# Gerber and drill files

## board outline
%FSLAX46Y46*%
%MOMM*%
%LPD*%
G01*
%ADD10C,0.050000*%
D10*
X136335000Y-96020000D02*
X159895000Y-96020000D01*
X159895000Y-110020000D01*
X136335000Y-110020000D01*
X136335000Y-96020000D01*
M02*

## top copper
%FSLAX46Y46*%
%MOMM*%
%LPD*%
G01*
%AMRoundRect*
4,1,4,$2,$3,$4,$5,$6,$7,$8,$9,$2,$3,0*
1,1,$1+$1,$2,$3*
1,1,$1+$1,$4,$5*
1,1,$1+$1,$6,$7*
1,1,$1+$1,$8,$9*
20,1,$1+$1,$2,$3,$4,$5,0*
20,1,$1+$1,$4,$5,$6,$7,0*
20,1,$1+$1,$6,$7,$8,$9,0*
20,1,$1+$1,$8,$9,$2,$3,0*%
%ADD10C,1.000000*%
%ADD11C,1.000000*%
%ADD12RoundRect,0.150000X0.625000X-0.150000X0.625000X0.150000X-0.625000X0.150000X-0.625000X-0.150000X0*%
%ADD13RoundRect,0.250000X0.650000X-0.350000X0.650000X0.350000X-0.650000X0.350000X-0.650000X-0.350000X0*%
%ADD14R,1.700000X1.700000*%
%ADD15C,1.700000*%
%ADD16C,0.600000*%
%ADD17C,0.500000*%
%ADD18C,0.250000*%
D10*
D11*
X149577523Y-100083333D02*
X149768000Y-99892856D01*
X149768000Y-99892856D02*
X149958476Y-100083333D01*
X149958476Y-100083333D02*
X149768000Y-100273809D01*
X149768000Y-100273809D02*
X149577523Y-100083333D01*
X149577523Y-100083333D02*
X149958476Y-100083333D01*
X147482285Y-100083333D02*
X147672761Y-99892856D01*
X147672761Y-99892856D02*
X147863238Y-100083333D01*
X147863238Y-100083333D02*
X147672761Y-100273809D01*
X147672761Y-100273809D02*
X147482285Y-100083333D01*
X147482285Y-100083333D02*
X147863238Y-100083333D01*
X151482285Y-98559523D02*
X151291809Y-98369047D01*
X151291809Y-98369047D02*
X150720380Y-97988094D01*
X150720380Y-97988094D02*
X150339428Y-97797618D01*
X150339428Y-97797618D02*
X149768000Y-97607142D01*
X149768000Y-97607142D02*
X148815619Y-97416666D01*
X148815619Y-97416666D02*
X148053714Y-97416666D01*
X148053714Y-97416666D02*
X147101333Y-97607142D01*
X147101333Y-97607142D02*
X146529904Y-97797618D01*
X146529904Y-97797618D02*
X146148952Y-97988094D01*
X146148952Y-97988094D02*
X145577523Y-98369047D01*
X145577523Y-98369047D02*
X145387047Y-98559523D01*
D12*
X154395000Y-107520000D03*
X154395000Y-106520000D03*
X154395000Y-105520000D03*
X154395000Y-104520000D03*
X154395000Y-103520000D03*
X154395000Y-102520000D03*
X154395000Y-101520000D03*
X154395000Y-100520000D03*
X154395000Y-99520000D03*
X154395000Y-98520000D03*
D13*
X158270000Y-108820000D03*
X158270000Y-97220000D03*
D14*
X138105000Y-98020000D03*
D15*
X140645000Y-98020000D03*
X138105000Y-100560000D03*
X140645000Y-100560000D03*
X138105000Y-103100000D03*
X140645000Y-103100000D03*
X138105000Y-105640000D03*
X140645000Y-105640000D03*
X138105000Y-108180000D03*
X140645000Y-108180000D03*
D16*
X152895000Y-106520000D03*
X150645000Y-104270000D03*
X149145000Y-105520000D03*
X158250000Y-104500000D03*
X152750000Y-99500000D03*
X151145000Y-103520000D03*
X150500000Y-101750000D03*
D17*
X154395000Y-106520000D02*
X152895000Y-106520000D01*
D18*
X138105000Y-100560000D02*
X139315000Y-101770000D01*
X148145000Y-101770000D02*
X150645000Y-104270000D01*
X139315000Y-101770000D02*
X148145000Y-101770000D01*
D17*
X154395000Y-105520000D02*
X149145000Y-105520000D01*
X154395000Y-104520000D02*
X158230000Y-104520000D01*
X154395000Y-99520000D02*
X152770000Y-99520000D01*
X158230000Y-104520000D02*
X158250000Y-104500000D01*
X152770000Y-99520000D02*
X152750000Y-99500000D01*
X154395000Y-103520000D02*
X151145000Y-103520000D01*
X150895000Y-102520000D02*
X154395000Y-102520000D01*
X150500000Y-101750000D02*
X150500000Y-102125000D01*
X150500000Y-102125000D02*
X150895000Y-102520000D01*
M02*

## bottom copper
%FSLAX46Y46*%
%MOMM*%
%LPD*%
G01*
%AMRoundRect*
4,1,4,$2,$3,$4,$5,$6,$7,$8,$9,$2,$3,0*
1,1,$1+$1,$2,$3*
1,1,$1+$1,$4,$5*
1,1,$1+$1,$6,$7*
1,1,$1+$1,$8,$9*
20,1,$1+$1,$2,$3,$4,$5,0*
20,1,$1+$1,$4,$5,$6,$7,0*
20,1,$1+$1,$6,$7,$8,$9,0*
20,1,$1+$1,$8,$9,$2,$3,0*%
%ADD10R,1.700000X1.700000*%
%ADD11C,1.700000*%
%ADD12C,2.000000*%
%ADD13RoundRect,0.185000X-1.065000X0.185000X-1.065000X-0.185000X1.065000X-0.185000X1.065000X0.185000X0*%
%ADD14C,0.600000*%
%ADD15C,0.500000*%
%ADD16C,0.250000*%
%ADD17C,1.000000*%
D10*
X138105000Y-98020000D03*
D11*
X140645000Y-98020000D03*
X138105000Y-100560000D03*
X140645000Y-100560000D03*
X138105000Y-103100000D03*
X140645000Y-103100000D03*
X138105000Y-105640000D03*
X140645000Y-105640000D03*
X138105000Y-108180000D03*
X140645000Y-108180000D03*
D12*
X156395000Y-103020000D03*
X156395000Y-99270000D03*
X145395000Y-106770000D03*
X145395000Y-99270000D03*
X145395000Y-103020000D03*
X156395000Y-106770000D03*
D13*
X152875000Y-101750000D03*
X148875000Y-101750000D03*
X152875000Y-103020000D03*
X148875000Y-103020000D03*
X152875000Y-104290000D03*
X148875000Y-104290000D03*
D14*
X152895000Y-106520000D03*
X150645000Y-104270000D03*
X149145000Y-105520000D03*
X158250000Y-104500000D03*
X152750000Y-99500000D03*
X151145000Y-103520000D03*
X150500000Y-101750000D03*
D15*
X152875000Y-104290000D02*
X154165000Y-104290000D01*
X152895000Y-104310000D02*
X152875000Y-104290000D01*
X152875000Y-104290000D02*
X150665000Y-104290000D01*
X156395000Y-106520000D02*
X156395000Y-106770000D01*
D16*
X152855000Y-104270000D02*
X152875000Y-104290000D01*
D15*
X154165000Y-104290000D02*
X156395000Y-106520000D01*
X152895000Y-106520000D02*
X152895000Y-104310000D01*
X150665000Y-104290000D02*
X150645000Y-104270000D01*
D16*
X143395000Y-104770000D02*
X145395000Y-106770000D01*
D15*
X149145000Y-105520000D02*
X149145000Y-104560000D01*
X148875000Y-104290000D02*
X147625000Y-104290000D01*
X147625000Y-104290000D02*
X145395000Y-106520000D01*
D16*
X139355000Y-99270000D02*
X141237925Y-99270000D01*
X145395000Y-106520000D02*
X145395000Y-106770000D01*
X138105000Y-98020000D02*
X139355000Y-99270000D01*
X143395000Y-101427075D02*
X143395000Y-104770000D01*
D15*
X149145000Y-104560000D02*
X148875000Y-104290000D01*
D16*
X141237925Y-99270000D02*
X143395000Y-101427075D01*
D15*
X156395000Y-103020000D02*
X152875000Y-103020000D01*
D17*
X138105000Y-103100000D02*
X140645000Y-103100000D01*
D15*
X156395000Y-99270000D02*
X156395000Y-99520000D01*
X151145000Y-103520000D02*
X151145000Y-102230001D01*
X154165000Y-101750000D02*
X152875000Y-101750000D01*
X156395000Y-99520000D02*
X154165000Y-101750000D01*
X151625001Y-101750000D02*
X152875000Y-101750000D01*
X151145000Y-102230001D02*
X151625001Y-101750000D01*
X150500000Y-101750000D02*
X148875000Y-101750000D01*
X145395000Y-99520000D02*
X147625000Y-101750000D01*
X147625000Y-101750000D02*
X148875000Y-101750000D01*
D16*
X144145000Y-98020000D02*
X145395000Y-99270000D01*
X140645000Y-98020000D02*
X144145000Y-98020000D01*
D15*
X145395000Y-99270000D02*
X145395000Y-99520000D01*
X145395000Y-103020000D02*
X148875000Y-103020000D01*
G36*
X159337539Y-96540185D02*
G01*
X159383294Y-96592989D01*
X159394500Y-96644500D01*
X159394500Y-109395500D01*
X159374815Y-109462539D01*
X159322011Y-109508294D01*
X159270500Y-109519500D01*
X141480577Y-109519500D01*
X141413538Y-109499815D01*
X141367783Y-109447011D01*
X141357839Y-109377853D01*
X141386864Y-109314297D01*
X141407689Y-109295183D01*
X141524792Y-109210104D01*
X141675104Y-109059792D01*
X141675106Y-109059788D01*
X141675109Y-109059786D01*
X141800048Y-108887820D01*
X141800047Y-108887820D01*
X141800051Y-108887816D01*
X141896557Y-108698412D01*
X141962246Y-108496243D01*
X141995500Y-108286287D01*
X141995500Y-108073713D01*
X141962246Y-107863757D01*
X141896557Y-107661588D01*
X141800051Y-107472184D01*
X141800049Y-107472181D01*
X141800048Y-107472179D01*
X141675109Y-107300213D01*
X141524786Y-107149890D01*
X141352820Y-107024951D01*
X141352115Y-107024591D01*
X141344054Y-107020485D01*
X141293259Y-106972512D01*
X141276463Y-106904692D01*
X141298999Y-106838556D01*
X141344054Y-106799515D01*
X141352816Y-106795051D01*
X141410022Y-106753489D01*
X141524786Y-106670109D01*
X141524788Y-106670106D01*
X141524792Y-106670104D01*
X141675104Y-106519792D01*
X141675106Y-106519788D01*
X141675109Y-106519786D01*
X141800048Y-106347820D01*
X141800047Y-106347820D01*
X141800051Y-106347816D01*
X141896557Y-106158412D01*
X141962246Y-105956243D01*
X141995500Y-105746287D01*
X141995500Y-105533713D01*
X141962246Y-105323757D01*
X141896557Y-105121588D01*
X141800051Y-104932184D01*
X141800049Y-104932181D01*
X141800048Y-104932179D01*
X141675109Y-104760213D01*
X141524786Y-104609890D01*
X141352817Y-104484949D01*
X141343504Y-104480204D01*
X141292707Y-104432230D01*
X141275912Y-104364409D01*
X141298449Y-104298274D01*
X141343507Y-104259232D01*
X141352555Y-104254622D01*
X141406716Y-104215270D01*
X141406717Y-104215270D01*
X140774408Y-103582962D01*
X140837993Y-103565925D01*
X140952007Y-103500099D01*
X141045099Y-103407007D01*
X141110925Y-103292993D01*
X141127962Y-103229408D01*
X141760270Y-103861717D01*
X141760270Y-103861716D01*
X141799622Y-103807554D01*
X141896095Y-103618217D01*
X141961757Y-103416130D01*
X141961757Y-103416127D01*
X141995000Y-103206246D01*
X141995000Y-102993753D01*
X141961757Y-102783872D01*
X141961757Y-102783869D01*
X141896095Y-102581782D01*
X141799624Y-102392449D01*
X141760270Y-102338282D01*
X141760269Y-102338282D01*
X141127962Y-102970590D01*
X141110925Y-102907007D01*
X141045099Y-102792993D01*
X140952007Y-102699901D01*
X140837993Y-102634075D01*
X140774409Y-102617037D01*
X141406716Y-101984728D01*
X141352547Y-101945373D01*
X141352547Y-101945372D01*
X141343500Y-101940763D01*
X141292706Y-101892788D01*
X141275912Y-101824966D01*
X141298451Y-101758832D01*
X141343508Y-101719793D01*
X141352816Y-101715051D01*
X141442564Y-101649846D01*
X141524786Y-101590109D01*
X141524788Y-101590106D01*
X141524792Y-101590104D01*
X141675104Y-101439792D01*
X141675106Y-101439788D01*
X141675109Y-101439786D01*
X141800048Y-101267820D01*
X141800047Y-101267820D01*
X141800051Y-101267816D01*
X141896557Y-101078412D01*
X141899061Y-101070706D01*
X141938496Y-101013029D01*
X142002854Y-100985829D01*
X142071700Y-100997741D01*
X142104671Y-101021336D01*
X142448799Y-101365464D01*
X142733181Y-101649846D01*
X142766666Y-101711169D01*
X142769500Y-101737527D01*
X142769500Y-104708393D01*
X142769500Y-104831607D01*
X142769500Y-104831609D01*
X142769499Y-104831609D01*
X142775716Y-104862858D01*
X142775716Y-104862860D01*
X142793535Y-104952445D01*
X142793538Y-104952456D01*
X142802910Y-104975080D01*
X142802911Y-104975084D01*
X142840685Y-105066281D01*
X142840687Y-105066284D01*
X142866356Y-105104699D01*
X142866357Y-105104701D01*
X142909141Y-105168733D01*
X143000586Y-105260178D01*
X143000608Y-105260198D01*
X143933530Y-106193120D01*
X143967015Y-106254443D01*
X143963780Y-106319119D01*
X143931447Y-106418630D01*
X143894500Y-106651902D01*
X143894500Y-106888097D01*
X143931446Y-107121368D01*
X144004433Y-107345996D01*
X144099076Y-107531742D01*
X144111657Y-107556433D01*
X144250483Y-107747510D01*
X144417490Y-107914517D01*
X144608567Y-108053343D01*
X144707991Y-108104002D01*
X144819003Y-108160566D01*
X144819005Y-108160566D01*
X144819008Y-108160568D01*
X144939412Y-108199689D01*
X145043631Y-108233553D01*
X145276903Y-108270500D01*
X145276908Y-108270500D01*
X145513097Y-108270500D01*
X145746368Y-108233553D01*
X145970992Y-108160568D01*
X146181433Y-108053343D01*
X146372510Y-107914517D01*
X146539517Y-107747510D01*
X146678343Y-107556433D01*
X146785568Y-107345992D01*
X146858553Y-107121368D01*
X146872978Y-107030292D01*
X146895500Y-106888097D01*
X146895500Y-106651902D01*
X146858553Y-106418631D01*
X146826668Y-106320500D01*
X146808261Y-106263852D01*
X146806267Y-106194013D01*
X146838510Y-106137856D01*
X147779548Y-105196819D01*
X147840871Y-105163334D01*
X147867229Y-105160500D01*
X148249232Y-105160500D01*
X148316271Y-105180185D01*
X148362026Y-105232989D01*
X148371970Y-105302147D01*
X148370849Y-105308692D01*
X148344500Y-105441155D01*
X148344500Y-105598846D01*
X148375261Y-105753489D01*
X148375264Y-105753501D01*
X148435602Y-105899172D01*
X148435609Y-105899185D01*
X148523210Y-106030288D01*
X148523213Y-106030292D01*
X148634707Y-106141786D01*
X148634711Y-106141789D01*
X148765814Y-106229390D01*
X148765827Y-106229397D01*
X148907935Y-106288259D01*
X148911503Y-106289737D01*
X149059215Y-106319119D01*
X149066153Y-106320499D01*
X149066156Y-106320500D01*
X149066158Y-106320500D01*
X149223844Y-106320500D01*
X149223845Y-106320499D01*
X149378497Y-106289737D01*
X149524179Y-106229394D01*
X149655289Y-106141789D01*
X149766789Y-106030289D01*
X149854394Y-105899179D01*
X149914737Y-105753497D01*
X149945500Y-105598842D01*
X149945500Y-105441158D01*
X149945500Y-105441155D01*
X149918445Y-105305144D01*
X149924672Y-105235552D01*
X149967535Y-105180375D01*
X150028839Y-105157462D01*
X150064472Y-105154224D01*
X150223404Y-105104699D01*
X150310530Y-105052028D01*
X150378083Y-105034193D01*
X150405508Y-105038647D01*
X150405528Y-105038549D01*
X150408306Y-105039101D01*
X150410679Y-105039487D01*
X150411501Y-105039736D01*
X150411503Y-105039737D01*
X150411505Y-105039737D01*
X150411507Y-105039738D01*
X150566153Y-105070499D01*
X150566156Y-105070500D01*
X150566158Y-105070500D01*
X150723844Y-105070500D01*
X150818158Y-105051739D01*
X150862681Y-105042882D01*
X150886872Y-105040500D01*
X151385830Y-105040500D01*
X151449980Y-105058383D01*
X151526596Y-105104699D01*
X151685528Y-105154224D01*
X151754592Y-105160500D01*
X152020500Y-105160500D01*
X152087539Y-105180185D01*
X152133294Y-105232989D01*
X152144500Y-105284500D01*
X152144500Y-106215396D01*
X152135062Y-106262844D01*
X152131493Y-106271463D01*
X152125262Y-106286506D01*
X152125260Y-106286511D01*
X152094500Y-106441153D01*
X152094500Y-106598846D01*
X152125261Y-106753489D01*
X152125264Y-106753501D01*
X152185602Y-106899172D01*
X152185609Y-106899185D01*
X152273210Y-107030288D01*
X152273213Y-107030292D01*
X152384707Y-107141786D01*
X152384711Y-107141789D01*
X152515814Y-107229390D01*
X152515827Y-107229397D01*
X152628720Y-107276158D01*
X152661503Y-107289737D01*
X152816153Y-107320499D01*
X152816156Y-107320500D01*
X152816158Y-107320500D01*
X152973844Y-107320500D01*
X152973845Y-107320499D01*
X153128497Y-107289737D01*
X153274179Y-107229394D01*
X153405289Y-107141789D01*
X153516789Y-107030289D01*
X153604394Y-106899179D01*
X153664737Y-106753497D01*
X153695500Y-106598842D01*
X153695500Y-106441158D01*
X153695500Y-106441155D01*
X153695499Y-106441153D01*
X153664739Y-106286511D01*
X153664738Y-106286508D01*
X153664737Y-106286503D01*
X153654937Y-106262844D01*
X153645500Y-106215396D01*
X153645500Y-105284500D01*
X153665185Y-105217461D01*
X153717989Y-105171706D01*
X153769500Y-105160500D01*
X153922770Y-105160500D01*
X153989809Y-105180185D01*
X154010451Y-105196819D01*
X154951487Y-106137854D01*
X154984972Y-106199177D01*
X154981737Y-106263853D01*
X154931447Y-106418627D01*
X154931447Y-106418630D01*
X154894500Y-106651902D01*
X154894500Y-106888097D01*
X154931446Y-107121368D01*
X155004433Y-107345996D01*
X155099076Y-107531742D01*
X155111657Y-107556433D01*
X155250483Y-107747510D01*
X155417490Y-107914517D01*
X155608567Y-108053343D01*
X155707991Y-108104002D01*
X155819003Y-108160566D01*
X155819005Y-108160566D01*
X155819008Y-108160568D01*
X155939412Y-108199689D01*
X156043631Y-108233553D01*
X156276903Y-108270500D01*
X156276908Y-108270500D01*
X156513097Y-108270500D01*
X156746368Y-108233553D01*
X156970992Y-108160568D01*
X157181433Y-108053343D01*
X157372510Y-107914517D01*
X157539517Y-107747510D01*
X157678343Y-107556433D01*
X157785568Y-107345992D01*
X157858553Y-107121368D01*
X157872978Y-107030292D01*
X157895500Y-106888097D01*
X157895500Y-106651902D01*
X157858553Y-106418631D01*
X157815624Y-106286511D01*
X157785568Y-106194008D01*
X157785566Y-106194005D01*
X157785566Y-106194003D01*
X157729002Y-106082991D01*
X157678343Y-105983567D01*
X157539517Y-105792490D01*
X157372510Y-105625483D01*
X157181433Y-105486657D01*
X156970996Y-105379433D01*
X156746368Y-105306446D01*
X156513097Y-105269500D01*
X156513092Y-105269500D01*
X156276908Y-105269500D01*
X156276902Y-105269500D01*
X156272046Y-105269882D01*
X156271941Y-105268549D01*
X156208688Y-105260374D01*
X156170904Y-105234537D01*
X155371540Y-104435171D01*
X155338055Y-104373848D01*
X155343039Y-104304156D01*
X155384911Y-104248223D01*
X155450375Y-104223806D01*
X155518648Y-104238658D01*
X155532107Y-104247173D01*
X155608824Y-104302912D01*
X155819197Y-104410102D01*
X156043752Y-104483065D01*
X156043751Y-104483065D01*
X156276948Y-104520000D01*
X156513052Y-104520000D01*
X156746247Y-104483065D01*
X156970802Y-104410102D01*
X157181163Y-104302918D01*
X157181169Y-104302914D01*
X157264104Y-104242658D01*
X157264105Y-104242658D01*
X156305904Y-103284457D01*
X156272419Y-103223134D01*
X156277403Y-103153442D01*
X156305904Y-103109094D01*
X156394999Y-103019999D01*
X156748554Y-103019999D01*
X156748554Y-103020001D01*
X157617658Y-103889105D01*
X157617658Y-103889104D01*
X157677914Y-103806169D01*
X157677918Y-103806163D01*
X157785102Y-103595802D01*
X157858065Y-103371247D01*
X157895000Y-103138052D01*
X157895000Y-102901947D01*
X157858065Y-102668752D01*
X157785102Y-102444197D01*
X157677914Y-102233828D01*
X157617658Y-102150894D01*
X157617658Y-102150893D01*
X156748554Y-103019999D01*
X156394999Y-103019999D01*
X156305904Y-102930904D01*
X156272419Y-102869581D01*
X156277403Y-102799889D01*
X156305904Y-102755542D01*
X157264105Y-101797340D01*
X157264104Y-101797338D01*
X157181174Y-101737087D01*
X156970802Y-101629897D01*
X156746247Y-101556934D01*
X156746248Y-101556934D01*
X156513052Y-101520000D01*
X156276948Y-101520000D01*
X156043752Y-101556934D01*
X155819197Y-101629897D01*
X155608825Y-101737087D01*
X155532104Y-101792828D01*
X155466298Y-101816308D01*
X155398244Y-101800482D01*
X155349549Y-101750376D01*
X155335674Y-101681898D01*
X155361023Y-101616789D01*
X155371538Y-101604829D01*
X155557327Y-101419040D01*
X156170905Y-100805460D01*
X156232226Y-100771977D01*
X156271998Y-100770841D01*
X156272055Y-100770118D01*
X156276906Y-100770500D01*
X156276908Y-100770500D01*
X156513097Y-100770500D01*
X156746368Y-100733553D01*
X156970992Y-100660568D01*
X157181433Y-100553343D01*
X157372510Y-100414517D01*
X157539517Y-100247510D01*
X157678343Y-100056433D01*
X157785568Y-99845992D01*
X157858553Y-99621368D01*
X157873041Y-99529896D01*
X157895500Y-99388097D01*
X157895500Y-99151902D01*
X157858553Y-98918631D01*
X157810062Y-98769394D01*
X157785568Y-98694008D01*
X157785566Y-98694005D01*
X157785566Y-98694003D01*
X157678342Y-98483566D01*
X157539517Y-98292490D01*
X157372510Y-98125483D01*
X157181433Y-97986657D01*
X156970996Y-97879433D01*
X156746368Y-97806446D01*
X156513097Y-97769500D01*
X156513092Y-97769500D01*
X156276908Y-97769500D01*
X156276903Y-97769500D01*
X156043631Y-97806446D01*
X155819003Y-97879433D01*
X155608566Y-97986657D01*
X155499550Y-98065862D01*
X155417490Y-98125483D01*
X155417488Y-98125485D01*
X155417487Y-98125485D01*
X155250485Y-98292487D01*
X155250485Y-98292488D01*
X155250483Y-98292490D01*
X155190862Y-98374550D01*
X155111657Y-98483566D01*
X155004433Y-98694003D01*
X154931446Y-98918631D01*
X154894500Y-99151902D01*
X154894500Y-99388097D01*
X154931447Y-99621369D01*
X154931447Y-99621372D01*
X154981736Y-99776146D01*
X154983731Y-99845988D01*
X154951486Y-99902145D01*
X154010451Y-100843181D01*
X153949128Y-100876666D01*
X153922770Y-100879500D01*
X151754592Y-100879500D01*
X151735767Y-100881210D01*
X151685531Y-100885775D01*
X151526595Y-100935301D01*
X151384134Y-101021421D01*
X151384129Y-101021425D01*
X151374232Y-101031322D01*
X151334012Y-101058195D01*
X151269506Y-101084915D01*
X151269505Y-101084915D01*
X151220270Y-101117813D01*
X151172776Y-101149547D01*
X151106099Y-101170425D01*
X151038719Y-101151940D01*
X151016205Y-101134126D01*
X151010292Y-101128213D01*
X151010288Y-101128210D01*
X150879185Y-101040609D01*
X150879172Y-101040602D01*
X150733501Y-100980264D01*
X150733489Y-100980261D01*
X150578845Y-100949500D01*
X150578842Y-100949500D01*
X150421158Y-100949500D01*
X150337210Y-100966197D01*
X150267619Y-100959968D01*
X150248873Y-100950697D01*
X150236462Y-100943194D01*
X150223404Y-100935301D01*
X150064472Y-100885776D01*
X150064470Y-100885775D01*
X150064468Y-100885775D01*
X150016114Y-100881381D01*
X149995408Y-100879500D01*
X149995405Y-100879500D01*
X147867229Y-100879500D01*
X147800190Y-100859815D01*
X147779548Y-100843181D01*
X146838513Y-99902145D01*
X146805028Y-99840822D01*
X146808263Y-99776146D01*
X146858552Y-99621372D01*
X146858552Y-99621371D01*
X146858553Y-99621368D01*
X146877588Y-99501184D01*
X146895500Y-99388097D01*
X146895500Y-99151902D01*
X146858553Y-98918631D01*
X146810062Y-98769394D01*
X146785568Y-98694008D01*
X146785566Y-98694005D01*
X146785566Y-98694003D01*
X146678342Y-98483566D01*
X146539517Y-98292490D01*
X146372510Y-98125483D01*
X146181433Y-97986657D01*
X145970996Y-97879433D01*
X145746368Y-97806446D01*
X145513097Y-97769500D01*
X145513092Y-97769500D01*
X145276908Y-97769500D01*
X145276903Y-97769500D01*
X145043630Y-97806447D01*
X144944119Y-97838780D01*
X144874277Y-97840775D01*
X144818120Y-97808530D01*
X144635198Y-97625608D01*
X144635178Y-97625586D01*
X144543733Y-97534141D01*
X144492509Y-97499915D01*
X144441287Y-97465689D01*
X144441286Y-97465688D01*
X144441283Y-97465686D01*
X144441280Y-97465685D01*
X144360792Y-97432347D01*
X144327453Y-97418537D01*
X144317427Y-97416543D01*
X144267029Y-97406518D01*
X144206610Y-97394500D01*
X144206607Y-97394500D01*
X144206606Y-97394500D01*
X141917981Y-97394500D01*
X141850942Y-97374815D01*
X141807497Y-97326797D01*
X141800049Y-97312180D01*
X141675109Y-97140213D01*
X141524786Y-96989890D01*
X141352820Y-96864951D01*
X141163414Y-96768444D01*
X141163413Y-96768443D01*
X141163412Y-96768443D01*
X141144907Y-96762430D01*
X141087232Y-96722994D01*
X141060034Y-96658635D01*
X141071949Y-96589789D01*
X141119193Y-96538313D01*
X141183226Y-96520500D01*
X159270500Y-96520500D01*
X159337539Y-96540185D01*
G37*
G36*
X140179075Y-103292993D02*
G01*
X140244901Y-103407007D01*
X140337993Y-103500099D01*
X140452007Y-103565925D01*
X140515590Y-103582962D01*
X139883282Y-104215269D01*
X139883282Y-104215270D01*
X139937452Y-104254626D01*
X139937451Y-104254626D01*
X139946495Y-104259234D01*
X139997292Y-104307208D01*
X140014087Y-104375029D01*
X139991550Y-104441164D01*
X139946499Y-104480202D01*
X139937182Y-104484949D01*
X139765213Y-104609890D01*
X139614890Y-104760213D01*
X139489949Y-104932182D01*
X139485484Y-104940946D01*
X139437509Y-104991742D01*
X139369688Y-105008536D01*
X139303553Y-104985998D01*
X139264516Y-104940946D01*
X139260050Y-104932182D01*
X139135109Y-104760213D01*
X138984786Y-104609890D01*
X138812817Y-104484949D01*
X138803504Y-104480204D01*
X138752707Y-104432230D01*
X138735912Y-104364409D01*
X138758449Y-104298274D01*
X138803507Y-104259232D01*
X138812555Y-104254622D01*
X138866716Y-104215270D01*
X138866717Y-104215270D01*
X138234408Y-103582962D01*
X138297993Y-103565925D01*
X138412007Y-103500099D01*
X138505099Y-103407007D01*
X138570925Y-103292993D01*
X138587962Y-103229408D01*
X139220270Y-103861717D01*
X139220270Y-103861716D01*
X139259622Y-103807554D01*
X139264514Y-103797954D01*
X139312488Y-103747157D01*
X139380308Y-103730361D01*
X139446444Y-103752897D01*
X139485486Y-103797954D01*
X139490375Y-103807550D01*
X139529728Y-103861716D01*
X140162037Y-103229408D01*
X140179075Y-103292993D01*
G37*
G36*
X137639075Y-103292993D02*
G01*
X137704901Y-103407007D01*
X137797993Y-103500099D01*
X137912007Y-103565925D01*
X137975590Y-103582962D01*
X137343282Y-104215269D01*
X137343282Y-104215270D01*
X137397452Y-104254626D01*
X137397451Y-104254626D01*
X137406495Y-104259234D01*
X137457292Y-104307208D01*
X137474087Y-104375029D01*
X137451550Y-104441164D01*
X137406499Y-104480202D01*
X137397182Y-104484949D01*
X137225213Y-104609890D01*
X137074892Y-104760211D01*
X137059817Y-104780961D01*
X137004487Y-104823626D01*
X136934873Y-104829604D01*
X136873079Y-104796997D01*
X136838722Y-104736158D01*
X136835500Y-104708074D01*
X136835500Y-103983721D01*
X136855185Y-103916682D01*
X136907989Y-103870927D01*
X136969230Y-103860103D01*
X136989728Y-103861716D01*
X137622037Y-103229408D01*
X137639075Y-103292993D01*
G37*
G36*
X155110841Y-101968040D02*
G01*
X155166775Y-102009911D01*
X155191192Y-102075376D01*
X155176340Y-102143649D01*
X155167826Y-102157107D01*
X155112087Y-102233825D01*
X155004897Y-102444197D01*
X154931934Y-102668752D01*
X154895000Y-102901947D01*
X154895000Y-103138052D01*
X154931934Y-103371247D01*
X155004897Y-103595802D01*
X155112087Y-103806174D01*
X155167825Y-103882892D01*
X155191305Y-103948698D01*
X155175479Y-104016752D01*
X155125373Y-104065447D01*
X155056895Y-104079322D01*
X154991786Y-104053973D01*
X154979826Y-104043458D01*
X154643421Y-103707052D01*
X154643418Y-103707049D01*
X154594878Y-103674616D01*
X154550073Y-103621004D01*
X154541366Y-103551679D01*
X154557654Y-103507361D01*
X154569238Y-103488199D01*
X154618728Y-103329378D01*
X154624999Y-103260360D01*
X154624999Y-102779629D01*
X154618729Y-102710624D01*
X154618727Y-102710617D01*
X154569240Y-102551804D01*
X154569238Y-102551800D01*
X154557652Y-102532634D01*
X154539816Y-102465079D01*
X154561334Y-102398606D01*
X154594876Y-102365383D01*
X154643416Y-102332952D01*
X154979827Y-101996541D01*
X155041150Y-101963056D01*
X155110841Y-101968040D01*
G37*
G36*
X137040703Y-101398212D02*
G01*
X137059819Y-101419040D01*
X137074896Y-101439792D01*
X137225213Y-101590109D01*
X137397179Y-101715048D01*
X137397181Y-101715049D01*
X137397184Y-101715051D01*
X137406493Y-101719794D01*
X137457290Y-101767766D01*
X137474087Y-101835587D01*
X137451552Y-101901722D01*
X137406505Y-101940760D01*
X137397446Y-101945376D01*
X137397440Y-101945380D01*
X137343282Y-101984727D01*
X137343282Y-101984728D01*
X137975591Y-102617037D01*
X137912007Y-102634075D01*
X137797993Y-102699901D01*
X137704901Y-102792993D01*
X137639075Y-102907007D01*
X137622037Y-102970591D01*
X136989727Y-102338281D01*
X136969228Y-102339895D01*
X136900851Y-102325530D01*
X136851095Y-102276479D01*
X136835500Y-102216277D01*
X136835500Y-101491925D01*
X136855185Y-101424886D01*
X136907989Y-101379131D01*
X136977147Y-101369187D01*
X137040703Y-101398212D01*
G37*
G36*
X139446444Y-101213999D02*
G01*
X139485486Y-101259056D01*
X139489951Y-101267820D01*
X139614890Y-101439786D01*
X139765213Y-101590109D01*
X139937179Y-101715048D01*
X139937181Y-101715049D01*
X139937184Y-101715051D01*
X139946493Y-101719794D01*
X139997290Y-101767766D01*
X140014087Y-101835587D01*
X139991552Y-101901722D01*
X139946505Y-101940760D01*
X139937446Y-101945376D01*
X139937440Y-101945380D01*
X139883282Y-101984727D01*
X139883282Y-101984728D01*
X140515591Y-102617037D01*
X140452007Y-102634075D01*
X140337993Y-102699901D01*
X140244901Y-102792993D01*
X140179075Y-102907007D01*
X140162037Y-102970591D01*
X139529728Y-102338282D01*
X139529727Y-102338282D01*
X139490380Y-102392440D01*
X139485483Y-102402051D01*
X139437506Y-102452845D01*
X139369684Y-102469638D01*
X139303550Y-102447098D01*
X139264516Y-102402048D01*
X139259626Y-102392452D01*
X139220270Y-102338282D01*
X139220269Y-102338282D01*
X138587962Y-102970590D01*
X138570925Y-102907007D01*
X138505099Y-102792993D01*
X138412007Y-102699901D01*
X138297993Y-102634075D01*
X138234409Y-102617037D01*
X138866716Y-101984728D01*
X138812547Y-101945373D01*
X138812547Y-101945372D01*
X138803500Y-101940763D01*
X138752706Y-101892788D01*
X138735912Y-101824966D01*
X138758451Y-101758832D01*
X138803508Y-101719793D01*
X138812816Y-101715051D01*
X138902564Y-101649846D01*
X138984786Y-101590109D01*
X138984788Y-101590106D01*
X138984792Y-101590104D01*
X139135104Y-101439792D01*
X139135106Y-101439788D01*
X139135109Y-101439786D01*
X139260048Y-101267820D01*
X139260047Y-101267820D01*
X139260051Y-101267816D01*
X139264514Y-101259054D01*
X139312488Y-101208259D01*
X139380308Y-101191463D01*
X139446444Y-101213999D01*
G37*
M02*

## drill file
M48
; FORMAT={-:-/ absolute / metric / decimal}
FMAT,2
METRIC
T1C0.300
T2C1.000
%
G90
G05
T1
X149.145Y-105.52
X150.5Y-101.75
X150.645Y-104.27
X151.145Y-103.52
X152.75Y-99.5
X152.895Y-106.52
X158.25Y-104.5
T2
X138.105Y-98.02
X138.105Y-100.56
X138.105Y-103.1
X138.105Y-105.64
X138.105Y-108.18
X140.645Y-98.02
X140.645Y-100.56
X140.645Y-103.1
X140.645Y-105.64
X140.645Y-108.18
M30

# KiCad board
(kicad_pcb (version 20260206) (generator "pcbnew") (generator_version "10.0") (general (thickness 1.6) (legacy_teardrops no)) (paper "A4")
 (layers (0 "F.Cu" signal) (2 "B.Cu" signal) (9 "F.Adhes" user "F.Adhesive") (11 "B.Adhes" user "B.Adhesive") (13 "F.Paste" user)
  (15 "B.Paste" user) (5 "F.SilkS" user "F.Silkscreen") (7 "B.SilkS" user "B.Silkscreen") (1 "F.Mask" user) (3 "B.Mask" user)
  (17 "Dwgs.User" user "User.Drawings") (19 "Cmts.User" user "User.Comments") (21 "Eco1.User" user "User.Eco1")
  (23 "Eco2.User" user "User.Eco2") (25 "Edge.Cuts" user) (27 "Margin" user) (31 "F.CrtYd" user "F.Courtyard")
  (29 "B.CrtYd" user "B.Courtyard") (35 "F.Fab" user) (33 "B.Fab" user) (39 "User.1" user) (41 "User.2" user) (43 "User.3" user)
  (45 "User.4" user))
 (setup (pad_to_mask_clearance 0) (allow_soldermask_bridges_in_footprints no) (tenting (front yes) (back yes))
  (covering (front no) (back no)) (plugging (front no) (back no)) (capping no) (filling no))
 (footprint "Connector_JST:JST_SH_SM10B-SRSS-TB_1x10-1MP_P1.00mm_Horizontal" (layer "F.Cu") (at 156.395 103.02 90)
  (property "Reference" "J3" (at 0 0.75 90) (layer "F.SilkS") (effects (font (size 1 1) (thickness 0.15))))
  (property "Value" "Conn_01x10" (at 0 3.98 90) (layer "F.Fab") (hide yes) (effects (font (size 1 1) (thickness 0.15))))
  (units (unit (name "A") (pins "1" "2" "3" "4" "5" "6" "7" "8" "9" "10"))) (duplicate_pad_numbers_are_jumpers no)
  (pad "1" smd roundrect (at -4.5 -2 90) (size 0.6 1.55) (layers "F.Cu" "F.Mask" "F.Paste") (roundrect_rratio 0.25)
   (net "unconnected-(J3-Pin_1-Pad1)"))
  (pad "2" smd roundrect (at -3.5 -2 90) (size 0.6 1.55) (layers "F.Cu" "F.Mask" "F.Paste") (roundrect_rratio 0.25) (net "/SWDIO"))
  (pad "3" smd roundrect (at -2.5 -2 90) (size 0.6 1.55) (layers "F.Cu" "F.Mask" "F.Paste") (roundrect_rratio 0.25) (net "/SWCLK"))
  (pad "4" smd roundrect (at -1.5 -2 90) (size 0.6 1.55) (layers "F.Cu" "F.Mask" "F.Paste") (roundrect_rratio 0.25) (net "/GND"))
  (pad "5" smd roundrect (at -0.5 -2 90) (size 0.6 1.55) (layers "F.Cu" "F.Mask" "F.Paste") (roundrect_rratio 0.25) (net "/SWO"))
  (pad "6" smd roundrect (at 0.5 -2 90) (size 0.6 1.55) (layers "F.Cu" "F.Mask" "F.Paste") (roundrect_rratio 0.25) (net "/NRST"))
  (pad "7" smd roundrect (at 1.5 -2 90) (size 0.6 1.55) (layers "F.Cu" "F.Mask" "F.Paste") (roundrect_rratio 0.25)
   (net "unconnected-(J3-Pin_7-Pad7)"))
  (pad "8" smd roundrect (at 2.5 -2 90) (size 0.6 1.55) (layers "F.Cu" "F.Mask" "F.Paste") (roundrect_rratio 0.25)
   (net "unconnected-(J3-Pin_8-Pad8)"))
  (pad "9" smd roundrect (at 3.5 -2 90) (size 0.6 1.55) (layers "F.Cu" "F.Mask" "F.Paste") (roundrect_rratio 0.25) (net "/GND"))
  (pad "10" smd roundrect (at 4.5 -2 90) (size 0.6 1.55) (layers "F.Cu" "F.Mask" "F.Paste") (roundrect_rratio 0.25)
   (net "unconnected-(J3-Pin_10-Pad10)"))
  (pad "MP" smd roundrect (at -5.8 1.875 90) (size 1.2 1.8) (layers "F.Cu" "F.Mask" "F.Paste") (roundrect_rratio 0.208333))
  (pad "MP" smd roundrect (at 5.8 1.875 90) (size 1.2 1.8) (layers "F.Cu" "F.Mask" "F.Paste") (roundrect_rratio 0.208333)))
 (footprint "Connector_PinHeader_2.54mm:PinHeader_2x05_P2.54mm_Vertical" (layer "F.Cu") (at 138.105 98.02)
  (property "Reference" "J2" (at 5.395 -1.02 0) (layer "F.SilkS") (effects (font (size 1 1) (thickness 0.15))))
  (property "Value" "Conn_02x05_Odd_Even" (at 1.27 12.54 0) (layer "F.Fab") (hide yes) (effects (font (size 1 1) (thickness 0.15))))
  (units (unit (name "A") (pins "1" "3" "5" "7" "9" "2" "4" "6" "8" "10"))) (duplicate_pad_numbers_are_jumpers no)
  (pad "1" thru_hole rect (at 0 0) (size 1.7 1.7) (drill 1) (layers "*.Cu" "*.Mask") (remove_unused_layers no) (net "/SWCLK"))
  (pad "2" thru_hole circle (at 2.54 0) (size 1.7 1.7) (drill 1) (layers "*.Cu" "*.Mask") (remove_unused_layers no) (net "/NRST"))
  (pad "3" thru_hole circle (at 0 2.54) (size 1.7 1.7) (drill 1) (layers "*.Cu" "*.Mask") (remove_unused_layers no) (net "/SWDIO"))
  (pad "4" thru_hole circle (at 2.54 2.54) (size 1.7 1.7) (drill 1) (layers "*.Cu" "*.Mask") (remove_unused_layers no)
   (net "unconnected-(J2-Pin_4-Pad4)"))
  (pad "5" thru_hole circle (at 0 5.08) (size 1.7 1.7) (drill 1) (layers "*.Cu" "*.Mask") (remove_unused_layers no) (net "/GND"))
  (pad "6" thru_hole circle (at 2.54 5.08) (size 1.7 1.7) (drill 1) (layers "*.Cu" "*.Mask") (remove_unused_layers no) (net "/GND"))
  (pad "7" thru_hole circle (at 0 7.62) (size 1.7 1.7) (drill 1) (layers "*.Cu" "*.Mask") (remove_unused_layers no)
   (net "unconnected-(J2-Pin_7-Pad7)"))
  (pad "8" thru_hole circle (at 2.54 7.62) (size 1.7 1.7) (drill 1) (layers "*.Cu" "*.Mask") (remove_unused_layers no)
   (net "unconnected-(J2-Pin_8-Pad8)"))
  (pad "9" thru_hole circle (at 0 10.16) (size 1.7 1.7) (drill 1) (layers "*.Cu" "*.Mask") (remove_unused_layers no)
   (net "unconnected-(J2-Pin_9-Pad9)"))
  (pad "10" thru_hole circle (at 2.54 10.16) (size 1.7 1.7) (drill 1) (layers "*.Cu" "*.Mask") (remove_unused_layers no)
   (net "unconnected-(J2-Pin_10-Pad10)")))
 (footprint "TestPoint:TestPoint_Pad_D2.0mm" (layer "B.Cu") (at 156.395 103.02 90)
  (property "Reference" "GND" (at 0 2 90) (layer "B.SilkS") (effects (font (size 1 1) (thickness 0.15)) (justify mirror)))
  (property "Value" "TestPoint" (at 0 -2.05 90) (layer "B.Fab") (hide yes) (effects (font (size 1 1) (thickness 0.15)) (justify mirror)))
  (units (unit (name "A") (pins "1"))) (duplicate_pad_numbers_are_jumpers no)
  (pad "1" smd circle (at 0 0 90) (size 2 2) (layers "B.Cu" "B.Mask") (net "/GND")))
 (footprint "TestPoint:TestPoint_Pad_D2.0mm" (layer "B.Cu") (at 156.395 99.27 90)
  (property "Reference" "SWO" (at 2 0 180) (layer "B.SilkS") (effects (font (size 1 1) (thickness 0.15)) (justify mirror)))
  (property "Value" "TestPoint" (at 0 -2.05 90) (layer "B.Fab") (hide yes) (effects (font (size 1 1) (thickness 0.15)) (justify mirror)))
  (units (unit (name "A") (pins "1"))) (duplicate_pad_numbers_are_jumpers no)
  (pad "1" smd circle (at 0 0 90) (size 2 2) (layers "B.Cu" "B.Mask") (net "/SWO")))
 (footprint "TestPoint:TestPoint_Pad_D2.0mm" (layer "B.Cu") (at 145.395 106.77 -90)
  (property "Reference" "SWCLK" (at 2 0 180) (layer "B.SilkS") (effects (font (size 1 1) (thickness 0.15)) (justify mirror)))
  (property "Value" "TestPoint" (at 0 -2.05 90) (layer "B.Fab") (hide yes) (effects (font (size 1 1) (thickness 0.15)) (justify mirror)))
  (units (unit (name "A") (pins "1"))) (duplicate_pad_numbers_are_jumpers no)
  (pad "1" smd circle (at 0 0 270) (size 2 2) (layers "B.Cu" "B.Mask") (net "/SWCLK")))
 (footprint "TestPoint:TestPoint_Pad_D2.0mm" (layer "B.Cu") (at 145.395 99.27 -90)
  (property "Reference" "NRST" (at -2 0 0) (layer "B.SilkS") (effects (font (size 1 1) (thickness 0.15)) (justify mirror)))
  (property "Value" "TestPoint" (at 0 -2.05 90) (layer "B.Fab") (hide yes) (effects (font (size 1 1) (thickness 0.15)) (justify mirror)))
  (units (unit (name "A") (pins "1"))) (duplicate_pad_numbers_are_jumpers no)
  (pad "1" smd circle (at 0 0 270) (size 2 2) (layers "B.Cu" "B.Mask") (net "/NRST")))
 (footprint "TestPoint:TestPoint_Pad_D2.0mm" (layer "B.Cu") (at 145.395 103.02 -90)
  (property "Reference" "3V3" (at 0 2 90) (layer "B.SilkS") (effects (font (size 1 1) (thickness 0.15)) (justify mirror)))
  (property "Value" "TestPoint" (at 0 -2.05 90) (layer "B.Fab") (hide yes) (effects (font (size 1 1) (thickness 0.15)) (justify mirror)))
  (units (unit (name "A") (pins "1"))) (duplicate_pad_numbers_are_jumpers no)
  (pad "1" smd circle (at 0 0 270) (size 2 2) (layers "B.Cu" "B.Mask") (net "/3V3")))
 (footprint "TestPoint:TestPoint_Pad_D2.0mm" (layer "B.Cu") (at 156.395 106.77 90)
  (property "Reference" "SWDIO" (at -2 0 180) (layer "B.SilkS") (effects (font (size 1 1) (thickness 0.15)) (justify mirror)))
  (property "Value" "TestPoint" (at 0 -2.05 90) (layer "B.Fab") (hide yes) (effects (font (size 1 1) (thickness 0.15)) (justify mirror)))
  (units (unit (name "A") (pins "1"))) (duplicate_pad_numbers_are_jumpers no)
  (pad "1" smd circle (at 0 0 90) (size 2 2) (layers "B.Cu" "B.Mask") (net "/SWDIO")))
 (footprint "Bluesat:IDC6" (layer "B.Cu") (at 150.875 103.02 -90)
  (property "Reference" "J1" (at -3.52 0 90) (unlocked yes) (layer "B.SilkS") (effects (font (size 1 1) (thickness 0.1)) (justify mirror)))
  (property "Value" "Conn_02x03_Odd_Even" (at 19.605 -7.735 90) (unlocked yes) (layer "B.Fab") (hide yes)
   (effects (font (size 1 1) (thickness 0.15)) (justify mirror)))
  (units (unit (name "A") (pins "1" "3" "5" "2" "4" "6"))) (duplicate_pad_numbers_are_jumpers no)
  (pad "1" smd roundrect (at -1.27 -2 270) (size 0.74 2.5) (layers "B.Cu" "B.Mask" "B.Paste") (roundrect_rratio 0.25) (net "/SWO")
   (thermal_bridge_angle 45))
  (pad "2" smd roundrect (at -1.27 2 270) (size 0.74 2.5) (layers "B.Cu" "B.Mask" "B.Paste") (roundrect_rratio 0.25) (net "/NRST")
   (thermal_bridge_angle 45))
  (pad "3" smd roundrect (at 0 -2 270) (size 0.74 2.5) (layers "B.Cu" "B.Mask" "B.Paste") (roundrect_rratio 0.25) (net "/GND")
   (thermal_bridge_angle 45))
  (pad "4" smd roundrect (at 0 2 270) (size 0.74 2.5) (layers "B.Cu" "B.Mask" "B.Paste") (roundrect_rratio 0.25) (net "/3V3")
   (thermal_bridge_angle 45))
  (pad "5" smd roundrect (at 1.27 -2 270) (size 0.74 2.5) (layers "B.Cu" "B.Mask" "B.Paste") (roundrect_rratio 0.25) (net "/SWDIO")
   (thermal_bridge_angle 45))
  (pad "6" smd roundrect (at 1.27 2 270) (size 0.74 2.5) (layers "B.Cu" "B.Mask" "B.Paste") (roundrect_rratio 0.25) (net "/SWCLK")
   (thermal_bridge_angle 45)))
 (gr_rect (start 136.335 96.02) (end 159.895 110.02) (stroke (width 0.05) (type default)) (fill no) (layer "Edge.Cuts"))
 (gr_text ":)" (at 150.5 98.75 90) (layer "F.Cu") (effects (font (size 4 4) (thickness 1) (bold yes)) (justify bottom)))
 (segment (start 154.395 106.52) (end 152.895 106.52) (width 0.5) (layer "F.Cu") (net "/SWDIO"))
 (segment (start 138.105 100.56) (end 139.315 101.77) (width 0.25) (layer "F.Cu") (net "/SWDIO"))
 (segment (start 148.145 101.77) (end 150.645 104.27) (width 0.25) (layer "F.Cu") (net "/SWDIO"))
 (segment (start 139.315 101.77) (end 148.145 101.77) (width 0.25) (layer "F.Cu") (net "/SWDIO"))
 (via (at 152.895 106.52) (size 0.6) (drill 0.3) (layers "F.Cu" "B.Cu") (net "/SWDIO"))
 (via (at 150.645 104.27) (size 0.6) (drill 0.3) (layers "F.Cu" "B.Cu") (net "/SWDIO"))
 (segment (start 152.875 104.29) (end 154.165 104.29) (width 0.5) (layer "B.Cu") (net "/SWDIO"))
 (segment (start 152.895 104.31) (end 152.875 104.29) (width 0.5) (layer "B.Cu") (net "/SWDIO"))
 (segment (start 152.875 104.29) (end 150.665 104.29) (width 0.5) (layer "B.Cu") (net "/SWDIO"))
 (segment (start 156.395 106.52) (end 156.395 106.77) (width 0.5) (layer "B.Cu") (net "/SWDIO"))
 (segment (start 152.855 104.27) (end 152.875 104.29) (width 0.25) (layer "B.Cu") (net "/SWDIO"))
 (segment (start 154.165 104.29) (end 156.395 106.52) (width 0.5) (layer "B.Cu") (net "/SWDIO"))
 (segment (start 152.895 106.52) (end 152.895 104.31) (width 0.5) (layer "B.Cu") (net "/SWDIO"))
 (segment (start 150.665 104.29) (end 150.645 104.27) (width 0.5) (layer "B.Cu") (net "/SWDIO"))
 (segment (start 154.395 105.52) (end 149.145 105.52) (width 0.5) (layer "F.Cu") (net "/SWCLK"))
 (via (at 149.145 105.52) (size 0.6) (drill 0.3) (layers "F.Cu" "B.Cu") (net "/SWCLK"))
 (segment (start 143.395 104.77) (end 145.395 106.77) (width 0.25) (layer "B.Cu") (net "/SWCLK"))
 (segment (start 149.145 105.52) (end 149.145 104.56) (width 0.5) (layer "B.Cu") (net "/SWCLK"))
 (segment (start 148.875 104.29) (end 147.625 104.29) (width 0.5) (layer "B.Cu") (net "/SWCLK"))
 (segment (start 147.625 104.29) (end 145.395 106.52) (width 0.5) (layer "B.Cu") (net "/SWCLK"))
 (segment (start 139.355 99.27) (end 141.237925 99.27) (width 0.25) (layer "B.Cu") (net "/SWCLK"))
 (segment (start 145.395 106.52) (end 145.395 106.77) (width 0.25) (layer "B.Cu") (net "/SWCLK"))
 (segment (start 138.105 98.02) (end 139.355 99.27) (width 0.25) (layer "B.Cu") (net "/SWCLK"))
 (segment (start 143.395 101.427075) (end 143.395 104.77) (width 0.25) (layer "B.Cu") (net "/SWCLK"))
 (segment (start 149.145 104.56) (end 148.875 104.29) (width 0.5) (layer "B.Cu") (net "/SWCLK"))
 (segment (start 141.237925 99.27) (end 143.395 101.427075) (width 0.25) (layer "B.Cu") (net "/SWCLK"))
 (segment (start 154.395 104.52) (end 158.23 104.52) (width 0.5) (layer "F.Cu") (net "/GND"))
 (segment (start 154.395 99.52) (end 152.77 99.52) (width 0.5) (layer "F.Cu") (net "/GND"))
 (segment (start 158.23 104.52) (end 158.25 104.5) (width 0.5) (layer "F.Cu") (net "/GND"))
 (segment (start 152.77 99.52) (end 152.75 99.5) (width 0.5) (layer "F.Cu") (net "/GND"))
 (via (at 158.25 104.5) (size 0.6) (drill 0.3) (layers "F.Cu" "B.Cu") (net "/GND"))
 (via (at 152.75 99.5) (size 0.6) (drill 0.3) (layers "F.Cu" "B.Cu") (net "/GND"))
 (segment (start 156.395 103.02) (end 152.875 103.02) (width 0.5) (layer "B.Cu") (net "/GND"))
 (segment (start 138.105 103.1) (end 140.645 103.1) (width 1) (layer "B.Cu") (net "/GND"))
 (segment (start 154.395 103.52) (end 151.145 103.52) (width 0.5) (layer "F.Cu") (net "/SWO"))
 (via (at 151.145 103.52) (size 0.6) (drill 0.3) (layers "F.Cu" "B.Cu") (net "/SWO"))
 (segment (start 156.395 99.27) (end 156.395 99.52) (width 0.5) (layer "B.Cu") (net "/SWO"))
 (segment (start 151.145 103.52) (end 151.145 102.230001) (width 0.5) (layer "B.Cu") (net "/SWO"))
 (segment (start 154.165 101.75) (end 152.875 101.75) (width 0.5) (layer "B.Cu") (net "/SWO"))
 (segment (start 156.395 99.52) (end 154.165 101.75) (width 0.5) (layer "B.Cu") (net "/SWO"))
 (segment (start 151.625001 101.75) (end 152.875 101.75) (width 0.5) (layer "B.Cu") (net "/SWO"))
 (segment (start 151.145 102.230001) (end 151.625001 101.75) (width 0.5) (layer "B.Cu") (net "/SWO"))
 (segment (start 150.895 102.52) (end 154.395 102.52) (width 0.5) (layer "F.Cu") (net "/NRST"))
 (segment (start 150.5 101.75) (end 150.5 102.125) (width 0.5) (layer "F.Cu") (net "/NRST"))
 (segment (start 150.5 102.125) (end 150.895 102.52) (width 0.5) (layer "F.Cu") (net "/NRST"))
 (via (at 150.5 101.75) (size 0.6) (drill 0.3) (layers "F.Cu" "B.Cu") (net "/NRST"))
 (segment (start 150.5 101.75) (end 148.875 101.75) (width 0.5) (layer "B.Cu") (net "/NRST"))
 (segment (start 145.395 99.52) (end 147.625 101.75) (width 0.5) (layer "B.Cu") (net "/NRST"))
 (segment (start 147.625 101.75) (end 148.875 101.75) (width 0.5) (layer "B.Cu") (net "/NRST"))
 (segment (start 144.145 98.02) (end 145.395 99.27) (width 0.25) (layer "B.Cu") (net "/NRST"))
 (segment (start 140.645 98.02) (end 144.145 98.02) (width 0.25) (layer "B.Cu") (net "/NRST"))
 (segment (start 145.395 99.27) (end 145.395 99.52) (width 0.5) (layer "B.Cu") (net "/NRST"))
 (segment (start 145.395 103.02) (end 148.875 103.02) (width 0.5) (layer "B.Cu") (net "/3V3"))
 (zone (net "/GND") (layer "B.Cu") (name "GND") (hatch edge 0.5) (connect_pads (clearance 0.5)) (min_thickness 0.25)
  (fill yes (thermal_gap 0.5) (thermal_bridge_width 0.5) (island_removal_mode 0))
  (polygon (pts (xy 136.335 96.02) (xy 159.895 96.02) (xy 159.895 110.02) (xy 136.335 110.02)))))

